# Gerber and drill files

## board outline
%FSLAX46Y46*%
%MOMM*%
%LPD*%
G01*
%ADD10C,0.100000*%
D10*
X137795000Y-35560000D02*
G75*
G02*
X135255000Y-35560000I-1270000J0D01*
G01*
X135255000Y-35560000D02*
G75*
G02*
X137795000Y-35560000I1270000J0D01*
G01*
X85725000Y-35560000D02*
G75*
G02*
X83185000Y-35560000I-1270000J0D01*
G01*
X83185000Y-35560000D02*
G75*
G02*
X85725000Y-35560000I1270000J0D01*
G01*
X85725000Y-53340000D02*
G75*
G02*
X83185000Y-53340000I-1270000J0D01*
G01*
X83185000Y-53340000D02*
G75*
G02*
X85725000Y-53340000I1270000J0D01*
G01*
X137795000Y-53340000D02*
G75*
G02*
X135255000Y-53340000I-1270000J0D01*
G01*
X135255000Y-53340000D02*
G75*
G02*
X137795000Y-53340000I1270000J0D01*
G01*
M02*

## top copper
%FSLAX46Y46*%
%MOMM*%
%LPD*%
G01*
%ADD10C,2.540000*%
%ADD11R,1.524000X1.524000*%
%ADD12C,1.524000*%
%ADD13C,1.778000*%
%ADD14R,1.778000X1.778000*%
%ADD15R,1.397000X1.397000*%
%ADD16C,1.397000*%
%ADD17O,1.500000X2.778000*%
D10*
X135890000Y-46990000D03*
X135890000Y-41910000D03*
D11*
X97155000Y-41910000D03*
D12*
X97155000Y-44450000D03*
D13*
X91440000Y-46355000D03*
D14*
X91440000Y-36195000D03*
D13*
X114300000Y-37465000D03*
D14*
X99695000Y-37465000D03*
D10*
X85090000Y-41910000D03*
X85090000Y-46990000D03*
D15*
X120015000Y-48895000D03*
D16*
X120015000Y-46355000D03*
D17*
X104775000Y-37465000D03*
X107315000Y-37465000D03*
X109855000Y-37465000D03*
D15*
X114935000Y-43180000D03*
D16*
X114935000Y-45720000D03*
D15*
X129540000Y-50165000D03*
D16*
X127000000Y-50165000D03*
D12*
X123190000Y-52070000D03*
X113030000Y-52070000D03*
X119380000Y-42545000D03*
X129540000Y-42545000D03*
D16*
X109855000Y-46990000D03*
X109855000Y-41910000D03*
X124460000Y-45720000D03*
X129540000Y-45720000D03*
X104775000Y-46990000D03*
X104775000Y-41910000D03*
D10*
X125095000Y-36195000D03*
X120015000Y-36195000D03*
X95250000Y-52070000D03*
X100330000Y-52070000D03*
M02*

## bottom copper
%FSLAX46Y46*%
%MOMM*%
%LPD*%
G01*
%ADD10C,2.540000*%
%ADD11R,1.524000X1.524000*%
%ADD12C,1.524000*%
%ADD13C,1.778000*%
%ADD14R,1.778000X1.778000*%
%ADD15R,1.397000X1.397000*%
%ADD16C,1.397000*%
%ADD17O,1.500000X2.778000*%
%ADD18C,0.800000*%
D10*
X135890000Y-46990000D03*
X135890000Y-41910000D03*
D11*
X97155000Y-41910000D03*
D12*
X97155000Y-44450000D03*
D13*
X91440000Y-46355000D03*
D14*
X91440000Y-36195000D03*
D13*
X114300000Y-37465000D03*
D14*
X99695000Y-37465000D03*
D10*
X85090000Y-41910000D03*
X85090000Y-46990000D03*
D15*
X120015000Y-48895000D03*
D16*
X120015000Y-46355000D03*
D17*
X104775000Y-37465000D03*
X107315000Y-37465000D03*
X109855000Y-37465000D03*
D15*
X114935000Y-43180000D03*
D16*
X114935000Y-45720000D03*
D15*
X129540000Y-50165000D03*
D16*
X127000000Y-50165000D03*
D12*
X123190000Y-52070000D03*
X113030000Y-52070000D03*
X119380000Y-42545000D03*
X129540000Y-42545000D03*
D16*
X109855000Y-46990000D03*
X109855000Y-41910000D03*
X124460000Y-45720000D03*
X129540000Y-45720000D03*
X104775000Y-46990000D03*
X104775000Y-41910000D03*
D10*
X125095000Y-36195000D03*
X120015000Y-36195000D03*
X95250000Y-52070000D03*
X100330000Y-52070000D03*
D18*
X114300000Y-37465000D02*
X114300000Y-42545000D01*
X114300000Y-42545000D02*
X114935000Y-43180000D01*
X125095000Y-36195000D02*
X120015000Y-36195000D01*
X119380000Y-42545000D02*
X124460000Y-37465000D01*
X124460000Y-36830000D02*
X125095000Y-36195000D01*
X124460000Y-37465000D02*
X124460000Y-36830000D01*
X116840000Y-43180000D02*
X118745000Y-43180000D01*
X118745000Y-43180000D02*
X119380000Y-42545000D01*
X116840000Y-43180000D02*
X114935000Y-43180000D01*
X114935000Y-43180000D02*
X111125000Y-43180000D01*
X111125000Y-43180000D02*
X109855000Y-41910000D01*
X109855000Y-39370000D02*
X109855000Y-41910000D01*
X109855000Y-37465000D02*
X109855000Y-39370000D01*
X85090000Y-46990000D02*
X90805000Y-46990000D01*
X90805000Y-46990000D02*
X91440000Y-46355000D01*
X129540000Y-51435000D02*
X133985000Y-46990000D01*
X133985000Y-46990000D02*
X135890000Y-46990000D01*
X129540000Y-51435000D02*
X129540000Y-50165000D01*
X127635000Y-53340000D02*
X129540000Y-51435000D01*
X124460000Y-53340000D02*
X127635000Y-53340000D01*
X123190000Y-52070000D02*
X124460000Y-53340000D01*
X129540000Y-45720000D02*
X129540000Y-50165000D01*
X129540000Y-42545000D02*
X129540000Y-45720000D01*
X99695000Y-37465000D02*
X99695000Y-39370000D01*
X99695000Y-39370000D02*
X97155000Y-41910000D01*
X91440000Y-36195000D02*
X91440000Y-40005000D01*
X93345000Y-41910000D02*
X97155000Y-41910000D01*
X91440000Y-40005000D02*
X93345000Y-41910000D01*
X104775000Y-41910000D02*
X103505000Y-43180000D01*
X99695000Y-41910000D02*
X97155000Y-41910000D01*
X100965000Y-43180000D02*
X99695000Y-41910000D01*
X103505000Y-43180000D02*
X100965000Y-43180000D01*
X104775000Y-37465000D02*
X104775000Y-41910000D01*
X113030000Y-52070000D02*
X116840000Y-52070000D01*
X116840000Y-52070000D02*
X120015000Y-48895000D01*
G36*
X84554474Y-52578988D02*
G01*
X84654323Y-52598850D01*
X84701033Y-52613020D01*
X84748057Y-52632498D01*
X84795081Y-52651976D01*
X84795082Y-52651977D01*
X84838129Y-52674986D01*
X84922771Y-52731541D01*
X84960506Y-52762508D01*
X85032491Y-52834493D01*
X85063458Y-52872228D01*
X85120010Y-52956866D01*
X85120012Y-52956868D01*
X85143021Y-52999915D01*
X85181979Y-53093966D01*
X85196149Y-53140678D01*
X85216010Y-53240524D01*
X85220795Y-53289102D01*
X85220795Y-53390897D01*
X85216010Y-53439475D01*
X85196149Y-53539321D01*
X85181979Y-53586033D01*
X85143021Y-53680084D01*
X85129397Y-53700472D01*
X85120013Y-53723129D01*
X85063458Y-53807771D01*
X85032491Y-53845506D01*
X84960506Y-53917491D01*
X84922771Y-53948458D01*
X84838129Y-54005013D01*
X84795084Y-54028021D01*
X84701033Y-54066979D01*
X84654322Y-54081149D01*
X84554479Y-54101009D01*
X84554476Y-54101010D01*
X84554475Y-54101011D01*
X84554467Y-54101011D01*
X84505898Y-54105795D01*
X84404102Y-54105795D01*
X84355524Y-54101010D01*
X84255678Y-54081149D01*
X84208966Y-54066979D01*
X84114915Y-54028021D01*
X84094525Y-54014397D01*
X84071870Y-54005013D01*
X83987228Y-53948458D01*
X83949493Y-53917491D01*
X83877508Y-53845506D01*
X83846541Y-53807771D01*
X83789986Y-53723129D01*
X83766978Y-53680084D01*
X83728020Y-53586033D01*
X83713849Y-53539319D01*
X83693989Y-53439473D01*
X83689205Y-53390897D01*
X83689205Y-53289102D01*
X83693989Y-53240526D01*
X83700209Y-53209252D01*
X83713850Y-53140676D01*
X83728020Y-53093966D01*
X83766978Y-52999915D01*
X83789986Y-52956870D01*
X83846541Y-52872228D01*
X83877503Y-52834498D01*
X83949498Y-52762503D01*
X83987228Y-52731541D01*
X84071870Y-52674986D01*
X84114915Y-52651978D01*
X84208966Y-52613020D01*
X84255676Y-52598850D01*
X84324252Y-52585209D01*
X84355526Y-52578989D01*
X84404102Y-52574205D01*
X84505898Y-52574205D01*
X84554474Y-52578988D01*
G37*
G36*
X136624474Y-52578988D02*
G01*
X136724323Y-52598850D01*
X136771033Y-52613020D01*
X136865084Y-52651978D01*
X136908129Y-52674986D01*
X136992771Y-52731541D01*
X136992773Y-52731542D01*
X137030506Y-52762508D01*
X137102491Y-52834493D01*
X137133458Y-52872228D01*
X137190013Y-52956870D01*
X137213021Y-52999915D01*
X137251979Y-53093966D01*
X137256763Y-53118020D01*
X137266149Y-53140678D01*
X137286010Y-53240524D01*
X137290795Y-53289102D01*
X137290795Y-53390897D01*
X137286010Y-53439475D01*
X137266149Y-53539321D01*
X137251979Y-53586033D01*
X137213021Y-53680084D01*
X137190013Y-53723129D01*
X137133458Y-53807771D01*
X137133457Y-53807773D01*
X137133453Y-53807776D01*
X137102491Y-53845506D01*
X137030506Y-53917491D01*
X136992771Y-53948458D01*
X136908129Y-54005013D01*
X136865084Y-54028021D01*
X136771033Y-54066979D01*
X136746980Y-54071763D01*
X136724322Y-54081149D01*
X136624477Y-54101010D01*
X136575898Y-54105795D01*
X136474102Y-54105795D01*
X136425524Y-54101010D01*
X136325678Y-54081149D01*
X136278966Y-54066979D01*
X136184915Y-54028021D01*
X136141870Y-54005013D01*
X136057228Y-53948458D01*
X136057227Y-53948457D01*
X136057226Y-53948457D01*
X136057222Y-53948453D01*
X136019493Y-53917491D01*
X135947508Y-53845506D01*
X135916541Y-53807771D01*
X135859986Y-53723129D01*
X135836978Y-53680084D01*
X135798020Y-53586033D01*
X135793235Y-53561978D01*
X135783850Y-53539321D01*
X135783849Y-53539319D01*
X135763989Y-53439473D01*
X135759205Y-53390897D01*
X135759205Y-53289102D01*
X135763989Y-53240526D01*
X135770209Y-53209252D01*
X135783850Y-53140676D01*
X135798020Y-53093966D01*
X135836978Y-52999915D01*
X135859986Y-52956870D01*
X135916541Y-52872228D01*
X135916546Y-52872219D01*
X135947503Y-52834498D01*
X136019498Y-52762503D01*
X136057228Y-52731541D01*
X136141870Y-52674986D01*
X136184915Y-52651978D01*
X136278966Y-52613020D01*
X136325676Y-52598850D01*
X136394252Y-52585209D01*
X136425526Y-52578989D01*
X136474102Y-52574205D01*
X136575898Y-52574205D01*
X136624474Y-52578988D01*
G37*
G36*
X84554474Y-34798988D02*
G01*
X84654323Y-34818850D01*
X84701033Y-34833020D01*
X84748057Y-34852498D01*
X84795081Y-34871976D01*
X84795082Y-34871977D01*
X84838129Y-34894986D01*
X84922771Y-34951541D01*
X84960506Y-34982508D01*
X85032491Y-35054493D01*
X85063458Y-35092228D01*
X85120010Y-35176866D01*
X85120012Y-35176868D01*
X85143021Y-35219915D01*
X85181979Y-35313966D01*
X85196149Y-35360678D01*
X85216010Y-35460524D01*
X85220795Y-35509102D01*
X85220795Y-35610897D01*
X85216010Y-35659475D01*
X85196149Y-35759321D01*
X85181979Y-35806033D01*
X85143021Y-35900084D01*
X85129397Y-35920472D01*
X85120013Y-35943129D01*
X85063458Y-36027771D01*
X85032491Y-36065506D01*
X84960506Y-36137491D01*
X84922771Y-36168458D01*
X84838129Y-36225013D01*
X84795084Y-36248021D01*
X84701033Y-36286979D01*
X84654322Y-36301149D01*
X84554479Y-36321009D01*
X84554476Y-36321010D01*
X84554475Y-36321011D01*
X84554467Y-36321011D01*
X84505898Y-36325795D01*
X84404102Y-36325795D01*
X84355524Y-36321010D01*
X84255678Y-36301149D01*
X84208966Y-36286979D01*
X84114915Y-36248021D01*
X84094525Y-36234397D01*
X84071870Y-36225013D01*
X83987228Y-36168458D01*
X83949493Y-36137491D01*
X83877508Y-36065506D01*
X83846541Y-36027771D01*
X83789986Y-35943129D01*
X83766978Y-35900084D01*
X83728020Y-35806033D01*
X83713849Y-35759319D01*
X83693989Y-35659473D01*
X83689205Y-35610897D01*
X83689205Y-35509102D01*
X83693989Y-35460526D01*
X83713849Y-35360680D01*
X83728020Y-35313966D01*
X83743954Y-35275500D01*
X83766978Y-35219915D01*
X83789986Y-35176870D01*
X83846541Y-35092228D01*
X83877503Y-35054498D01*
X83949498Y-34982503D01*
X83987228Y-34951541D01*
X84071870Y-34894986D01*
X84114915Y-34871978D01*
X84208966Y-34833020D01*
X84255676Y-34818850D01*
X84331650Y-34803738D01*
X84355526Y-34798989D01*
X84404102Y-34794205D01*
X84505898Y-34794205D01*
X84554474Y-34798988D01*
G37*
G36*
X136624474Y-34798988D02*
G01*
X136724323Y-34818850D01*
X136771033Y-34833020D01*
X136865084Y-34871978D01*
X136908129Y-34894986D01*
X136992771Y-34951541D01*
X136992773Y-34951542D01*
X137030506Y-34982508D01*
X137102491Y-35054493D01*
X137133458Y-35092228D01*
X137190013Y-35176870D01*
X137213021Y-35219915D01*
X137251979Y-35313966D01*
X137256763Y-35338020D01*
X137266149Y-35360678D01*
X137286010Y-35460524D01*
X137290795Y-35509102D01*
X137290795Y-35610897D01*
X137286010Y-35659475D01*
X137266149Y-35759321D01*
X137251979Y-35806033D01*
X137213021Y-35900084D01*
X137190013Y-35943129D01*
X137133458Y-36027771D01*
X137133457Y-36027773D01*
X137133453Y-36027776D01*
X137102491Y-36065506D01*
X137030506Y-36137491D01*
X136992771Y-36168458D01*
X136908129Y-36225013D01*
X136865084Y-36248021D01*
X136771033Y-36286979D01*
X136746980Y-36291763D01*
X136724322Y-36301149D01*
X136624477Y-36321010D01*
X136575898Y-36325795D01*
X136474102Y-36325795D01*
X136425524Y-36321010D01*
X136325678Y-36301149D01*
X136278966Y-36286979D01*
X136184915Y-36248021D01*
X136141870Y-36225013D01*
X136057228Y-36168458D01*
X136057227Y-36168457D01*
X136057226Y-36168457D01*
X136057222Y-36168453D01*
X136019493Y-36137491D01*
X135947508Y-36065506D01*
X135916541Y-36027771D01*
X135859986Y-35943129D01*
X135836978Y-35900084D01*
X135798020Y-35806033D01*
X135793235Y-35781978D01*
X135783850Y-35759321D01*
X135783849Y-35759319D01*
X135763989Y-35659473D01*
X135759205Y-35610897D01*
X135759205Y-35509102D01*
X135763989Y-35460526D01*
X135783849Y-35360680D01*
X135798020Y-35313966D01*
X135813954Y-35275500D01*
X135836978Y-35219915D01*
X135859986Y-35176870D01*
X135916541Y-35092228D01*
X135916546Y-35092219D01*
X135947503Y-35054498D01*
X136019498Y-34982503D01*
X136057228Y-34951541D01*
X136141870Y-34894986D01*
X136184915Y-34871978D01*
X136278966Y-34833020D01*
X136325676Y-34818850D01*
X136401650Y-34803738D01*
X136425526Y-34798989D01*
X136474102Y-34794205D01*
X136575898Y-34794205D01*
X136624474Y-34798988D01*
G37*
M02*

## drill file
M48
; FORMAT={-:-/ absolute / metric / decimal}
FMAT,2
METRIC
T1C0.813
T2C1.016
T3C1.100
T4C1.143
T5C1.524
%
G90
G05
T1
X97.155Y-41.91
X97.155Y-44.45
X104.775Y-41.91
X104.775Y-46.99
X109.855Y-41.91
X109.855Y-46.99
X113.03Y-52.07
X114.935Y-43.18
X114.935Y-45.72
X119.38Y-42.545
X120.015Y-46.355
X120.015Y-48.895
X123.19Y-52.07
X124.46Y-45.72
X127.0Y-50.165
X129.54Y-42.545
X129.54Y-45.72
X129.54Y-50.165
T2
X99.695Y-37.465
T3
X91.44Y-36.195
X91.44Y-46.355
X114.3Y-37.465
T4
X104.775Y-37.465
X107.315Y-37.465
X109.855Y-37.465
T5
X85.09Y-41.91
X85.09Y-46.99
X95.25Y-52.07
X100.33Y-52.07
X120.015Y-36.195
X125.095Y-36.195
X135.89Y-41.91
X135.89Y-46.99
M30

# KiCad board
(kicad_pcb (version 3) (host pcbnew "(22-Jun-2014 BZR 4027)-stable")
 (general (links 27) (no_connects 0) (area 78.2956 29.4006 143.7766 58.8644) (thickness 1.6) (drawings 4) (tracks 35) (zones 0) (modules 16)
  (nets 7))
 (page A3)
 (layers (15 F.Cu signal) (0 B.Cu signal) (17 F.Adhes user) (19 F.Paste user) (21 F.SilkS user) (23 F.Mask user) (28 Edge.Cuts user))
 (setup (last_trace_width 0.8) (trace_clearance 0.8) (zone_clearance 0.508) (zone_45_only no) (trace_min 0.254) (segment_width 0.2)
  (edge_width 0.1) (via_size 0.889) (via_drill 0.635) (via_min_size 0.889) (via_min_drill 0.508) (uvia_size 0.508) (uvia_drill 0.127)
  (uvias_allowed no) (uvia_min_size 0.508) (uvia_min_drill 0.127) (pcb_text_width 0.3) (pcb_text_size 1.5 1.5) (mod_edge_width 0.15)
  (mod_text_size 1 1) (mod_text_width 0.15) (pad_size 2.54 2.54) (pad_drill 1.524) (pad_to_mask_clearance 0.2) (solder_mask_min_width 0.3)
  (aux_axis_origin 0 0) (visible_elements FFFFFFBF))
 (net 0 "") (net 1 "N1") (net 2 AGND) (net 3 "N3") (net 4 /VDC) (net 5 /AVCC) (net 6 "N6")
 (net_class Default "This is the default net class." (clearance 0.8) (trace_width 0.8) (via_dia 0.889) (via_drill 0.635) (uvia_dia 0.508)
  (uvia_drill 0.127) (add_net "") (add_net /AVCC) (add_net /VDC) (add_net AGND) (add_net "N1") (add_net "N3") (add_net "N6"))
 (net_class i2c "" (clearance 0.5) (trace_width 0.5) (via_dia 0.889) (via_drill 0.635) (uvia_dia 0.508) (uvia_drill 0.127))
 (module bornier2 (layer F.Cu) (at 135.89 44.45 90)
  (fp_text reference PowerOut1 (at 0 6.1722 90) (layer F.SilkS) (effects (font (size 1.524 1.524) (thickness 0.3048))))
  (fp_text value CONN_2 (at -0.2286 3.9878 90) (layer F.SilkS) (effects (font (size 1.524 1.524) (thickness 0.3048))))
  (pad 1 thru_hole circle (at -2.54 0 90) (size 2.54 2.54) (drill 1.524) (layers *.Cu *.Mask F.SilkS) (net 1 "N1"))
  (pad 2 thru_hole circle (at 2.54 0 90) (size 2.54 2.54) (drill 1.524) (layers *.Cu *.Mask F.SilkS) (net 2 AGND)))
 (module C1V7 (layer F.Cu) (at 97.155 43.18 270)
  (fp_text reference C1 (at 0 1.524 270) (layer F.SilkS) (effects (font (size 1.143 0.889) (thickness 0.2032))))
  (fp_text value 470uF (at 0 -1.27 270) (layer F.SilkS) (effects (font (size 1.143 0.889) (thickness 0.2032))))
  (pad 1 thru_hole rect (at -1.27 0 270) (size 1.524 1.524) (drill 0.8128) (layers *.Cu *.Mask F.SilkS) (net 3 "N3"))
  (pad 2 thru_hole circle (at 1.27 0 270) (size 1.524 1.524) (drill 0.8128) (layers *.Cu *.Mask F.SilkS) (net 2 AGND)))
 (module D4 (layer F.Cu) (at 91.44 41.275 90)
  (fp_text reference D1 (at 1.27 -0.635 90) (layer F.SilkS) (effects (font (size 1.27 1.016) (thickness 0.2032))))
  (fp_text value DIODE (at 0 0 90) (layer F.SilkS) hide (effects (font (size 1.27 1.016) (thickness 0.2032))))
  (pad 1 thru_hole circle (at -5.08 0 90) (size 1.778 1.778) (drill 1.1) (layers *.Cu *.Mask F.SilkS) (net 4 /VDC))
  (pad 2 thru_hole rect (at 5.08 0 90) (size 1.778 1.778) (drill 1.1) (layers *.Cu *.Mask F.SilkS) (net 3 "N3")))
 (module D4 (layer F.Cu) (at 107.315 37.465 180)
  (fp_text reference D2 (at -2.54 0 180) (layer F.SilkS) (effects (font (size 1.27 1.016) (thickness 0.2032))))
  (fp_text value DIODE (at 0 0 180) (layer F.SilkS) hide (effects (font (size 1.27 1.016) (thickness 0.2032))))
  (pad 1 thru_hole circle (at -6.985 0 180) (size 1.778 1.778) (drill 1.1) (layers *.Cu *.Mask F.SilkS) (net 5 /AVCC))
  (pad 2 thru_hole rect (at 7.62 0 180) (size 1.778 1.778) (drill 1.016) (layers *.Cu *.Mask F.SilkS) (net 3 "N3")))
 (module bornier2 (layer F.Cu) (at 85.09 44.45 270)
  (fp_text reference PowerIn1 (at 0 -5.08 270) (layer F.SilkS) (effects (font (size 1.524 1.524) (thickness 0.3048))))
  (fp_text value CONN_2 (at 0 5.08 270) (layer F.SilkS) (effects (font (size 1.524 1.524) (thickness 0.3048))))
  (pad 1 thru_hole circle (at -2.54 0 270) (size 2.54 2.54) (drill 1.524) (layers *.Cu *.Mask F.SilkS) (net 2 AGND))
  (pad 2 thru_hole circle (at 2.54 0 270) (size 2.54 2.54) (drill 1.524) (layers *.Cu *.Mask F.SilkS) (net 4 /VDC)))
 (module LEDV (layer F.Cu) (at 120.015 47.625 90)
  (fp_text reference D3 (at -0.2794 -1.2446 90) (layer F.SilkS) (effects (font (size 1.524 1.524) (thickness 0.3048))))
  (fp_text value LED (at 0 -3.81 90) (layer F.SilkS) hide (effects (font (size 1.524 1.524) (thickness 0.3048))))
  (pad 1 thru_hole rect (at -1.27 0 90) (size 1.397 1.397) (drill 0.8128) (layers *.Cu *.Mask F.SilkS) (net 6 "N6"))
  (pad 2 thru_hole circle (at 1.27 0 90) (size 1.397 1.397) (drill 0.8128) (layers *.Cu *.Mask F.SilkS) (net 2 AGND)))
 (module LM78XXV (layer B.Cu) (at 107.315 37.465 270)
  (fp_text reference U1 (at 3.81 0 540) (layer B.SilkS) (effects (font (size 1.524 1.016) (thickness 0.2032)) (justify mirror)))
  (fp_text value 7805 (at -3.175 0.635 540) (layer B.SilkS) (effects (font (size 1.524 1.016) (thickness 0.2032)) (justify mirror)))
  (pad VI thru_hole oval (at 0 2.54 270) (size 2.778 1.5) (drill 1.143) (layers *.Cu *.Mask) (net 3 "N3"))
  (pad GND thru_hole oval (at 0 0 270) (size 2.778 1.5) (drill 1.143) (layers *.Cu *.Mask) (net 2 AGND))
  (pad VO thru_hole oval (at 0 -2.54 270) (size 2.778 1.5) (drill 1.143) (layers *.Cu *.Mask) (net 5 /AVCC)))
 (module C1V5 (layer F.Cu) (at 114.935 44.45 270)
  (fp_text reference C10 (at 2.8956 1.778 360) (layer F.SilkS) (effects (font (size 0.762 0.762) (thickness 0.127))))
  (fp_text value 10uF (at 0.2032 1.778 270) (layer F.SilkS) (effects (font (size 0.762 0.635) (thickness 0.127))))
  (pad 1 thru_hole rect (at -1.27 0 270) (size 1.397 1.397) (drill 0.8128) (layers *.Cu *.Mask F.SilkS) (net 5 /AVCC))
  (pad 2 thru_hole circle (at 1.27 0 270) (size 1.397 1.397) (drill 0.8128) (layers *.Cu *.Mask F.SilkS) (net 2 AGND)))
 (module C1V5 (layer F.Cu) (at 128.27 50.165 180)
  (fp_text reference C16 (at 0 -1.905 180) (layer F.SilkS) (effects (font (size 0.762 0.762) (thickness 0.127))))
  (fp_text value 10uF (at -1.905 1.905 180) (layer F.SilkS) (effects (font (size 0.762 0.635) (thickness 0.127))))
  (pad 1 thru_hole rect (at -1.27 0 180) (size 1.397 1.397) (drill 0.8128) (layers *.Cu *.Mask F.SilkS) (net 1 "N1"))
  (pad 2 thru_hole circle (at 1.27 0 180) (size 1.397 1.397) (drill 0.8128) (layers *.Cu *.Mask F.SilkS) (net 2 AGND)))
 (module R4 (layer F.Cu) (at 118.11 52.07 180) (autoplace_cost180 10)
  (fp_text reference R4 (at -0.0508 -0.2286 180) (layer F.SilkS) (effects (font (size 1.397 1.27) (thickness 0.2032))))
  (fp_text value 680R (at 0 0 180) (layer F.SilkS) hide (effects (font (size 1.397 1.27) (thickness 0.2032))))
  (pad 1 thru_hole circle (at -5.08 0 180) (size 1.524 1.524) (drill 0.8128) (layers *.Cu *.Mask F.SilkS) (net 1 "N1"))
  (pad 2 thru_hole circle (at 5.08 0 180) (size 1.524 1.524) (drill 0.8128) (layers *.Cu *.Mask F.SilkS) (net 6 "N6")))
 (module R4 (layer F.Cu) (at 124.46 42.545) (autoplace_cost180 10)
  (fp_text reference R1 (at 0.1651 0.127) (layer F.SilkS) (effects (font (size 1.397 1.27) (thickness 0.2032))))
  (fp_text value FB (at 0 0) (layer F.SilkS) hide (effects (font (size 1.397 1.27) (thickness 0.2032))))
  (pad 1 thru_hole circle (at -5.08 0) (size 1.524 1.524) (drill 0.8128) (layers *.Cu *.Mask F.SilkS) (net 5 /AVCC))
  (pad 2 thru_hole circle (at 5.08 0) (size 1.524 1.524) (drill 0.8128) (layers *.Cu *.Mask F.SilkS) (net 1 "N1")))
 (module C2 (layer F.Cu) (at 109.855 44.45 90)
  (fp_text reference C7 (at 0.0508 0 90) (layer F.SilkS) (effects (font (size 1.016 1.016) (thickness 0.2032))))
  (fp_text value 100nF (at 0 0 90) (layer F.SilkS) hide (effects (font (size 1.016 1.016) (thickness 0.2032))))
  (pad 1 thru_hole circle (at -2.54 0 90) (size 1.397 1.397) (drill 0.8128) (layers *.Cu *.Mask F.SilkS) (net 2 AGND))
  (pad 2 thru_hole circle (at 2.54 0 90) (size 1.397 1.397) (drill 0.8128) (layers *.Cu *.Mask F.SilkS) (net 5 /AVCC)))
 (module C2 (layer F.Cu) (at 127 45.72)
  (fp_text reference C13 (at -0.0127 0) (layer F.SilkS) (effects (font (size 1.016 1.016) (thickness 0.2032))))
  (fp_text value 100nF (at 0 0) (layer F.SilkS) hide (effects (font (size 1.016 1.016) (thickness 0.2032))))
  (pad 1 thru_hole circle (at -2.54 0) (size 1.397 1.397) (drill 0.8128) (layers *.Cu *.Mask F.SilkS) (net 2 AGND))
  (pad 2 thru_hole circle (at 2.54 0) (size 1.397 1.397) (drill 0.8128) (layers *.Cu *.Mask F.SilkS) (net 1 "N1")))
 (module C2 (layer F.Cu) (at 104.775 44.45 90)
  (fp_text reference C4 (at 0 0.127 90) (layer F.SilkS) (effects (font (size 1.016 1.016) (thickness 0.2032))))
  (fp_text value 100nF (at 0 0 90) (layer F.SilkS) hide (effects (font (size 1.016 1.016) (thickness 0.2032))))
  (pad 1 thru_hole circle (at -2.54 0 90) (size 1.397 1.397) (drill 0.8128) (layers *.Cu *.Mask F.SilkS) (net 2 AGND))
  (pad 2 thru_hole circle (at 2.54 0 90) (size 1.397 1.397) (drill 0.8128) (layers *.Cu *.Mask F.SilkS) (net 3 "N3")))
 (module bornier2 (layer F.Cu) (at 122.555 36.195 180)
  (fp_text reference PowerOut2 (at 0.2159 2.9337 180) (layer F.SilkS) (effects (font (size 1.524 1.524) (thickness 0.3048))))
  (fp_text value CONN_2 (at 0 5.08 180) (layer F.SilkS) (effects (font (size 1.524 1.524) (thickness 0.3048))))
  (pad 1 thru_hole circle (at -2.54 0 180) (size 2.54 2.54) (drill 1.524) (layers *.Cu *.Mask F.SilkS) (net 5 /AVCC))
  (pad 2 thru_hole circle (at 2.54 0 180) (size 2.54 2.54) (drill 1.524) (layers *.Cu *.Mask F.SilkS) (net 5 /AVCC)))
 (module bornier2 (layer F.Cu) (at 97.79 52.07)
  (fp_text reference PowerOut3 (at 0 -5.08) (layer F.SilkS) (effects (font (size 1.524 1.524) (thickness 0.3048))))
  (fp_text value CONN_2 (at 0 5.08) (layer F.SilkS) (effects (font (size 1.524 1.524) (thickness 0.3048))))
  (pad 1 thru_hole circle (at -2.54 0) (size 2.54 2.54) (drill 1.524) (layers *.Cu *.Mask F.SilkS) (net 2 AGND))
  (pad 2 thru_hole circle (at 2.54 0) (size 2.54 2.54) (drill 1.524) (layers *.Cu *.Mask F.SilkS) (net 2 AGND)))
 (gr_circle (center 136.525 35.56) (end 137.795 35.56) (layer Edge.Cuts) (width 0.1))
 (gr_circle (center 84.455 35.56) (end 85.725 35.56) (layer Edge.Cuts) (width 0.1))
 (gr_circle (center 84.455 53.34) (end 85.725 53.34) (layer Edge.Cuts) (width 0.1))
 (gr_circle (center 136.525 53.34) (end 137.795 53.34) (layer Edge.Cuts) (width 0.1))
 (segment (start 114.3 37.465) (end 114.3 42.545) (width 0.8) (layer B.Cu) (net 5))
 (segment (start 114.3 42.545) (end 114.935 43.18) (width 0.8) (layer B.Cu) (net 5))
 (segment (start 125.095 36.195) (end 120.015 36.195) (width 0.8) (layer B.Cu) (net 5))
 (segment (start 119.38 42.545) (end 124.46 37.465) (width 0.8) (layer B.Cu) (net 5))
 (segment (start 124.46 36.83) (end 125.095 36.195) (width 0.8) (layer B.Cu) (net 5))
 (segment (start 124.46 37.465) (end 124.46 36.83) (width 0.8) (layer B.Cu) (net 5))
 (segment (start 116.84 43.18) (end 118.745 43.18) (width 0.8) (layer B.Cu) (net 5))
 (segment (start 118.745 43.18) (end 119.38 42.545) (width 0.8) (layer B.Cu) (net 5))
 (segment (start 116.84 43.18) (end 114.935 43.18) (width 0.8) (layer B.Cu) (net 5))
 (segment (start 114.935 43.18) (end 111.125 43.18) (width 0.8) (layer B.Cu) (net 5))
 (segment (start 111.125 43.18) (end 109.855 41.91) (width 0.8) (layer B.Cu) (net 5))
 (segment (start 109.855 39.37) (end 109.855 41.91) (width 0.8) (layer B.Cu) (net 5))
 (segment (start 109.855 37.465) (end 109.855 39.37) (width 0.8) (layer B.Cu) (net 5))
 (segment (start 85.09 46.99) (end 90.805 46.99) (width 0.8) (layer B.Cu) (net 4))
 (segment (start 90.805 46.99) (end 91.44 46.355) (width 0.8) (layer B.Cu) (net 4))
 (segment (start 129.54 51.435) (end 133.985 46.99) (width 0.8) (layer B.Cu) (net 1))
 (segment (start 133.985 46.99) (end 135.89 46.99) (width 0.8) (layer B.Cu) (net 1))
 (segment (start 129.54 51.435) (end 129.54 50.165) (width 0.8) (layer B.Cu) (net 1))
 (segment (start 127.635 53.34) (end 129.54 51.435) (width 0.8) (layer B.Cu) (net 1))
 (segment (start 124.46 53.34) (end 127.635 53.34) (width 0.8) (layer B.Cu) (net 1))
 (segment (start 123.19 52.07) (end 124.46 53.34) (width 0.8) (layer B.Cu) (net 1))
 (segment (start 129.54 45.72) (end 129.54 50.165) (width 0.8) (layer B.Cu) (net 1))
 (segment (start 129.54 42.545) (end 129.54 45.72) (width 0.8) (layer B.Cu) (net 1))
 (segment (start 99.695 37.465) (end 99.695 39.37) (width 0.8) (layer B.Cu) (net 3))
 (segment (start 99.695 39.37) (end 97.155 41.91) (width 0.8) (layer B.Cu) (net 3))
 (segment (start 91.44 36.195) (end 91.44 40.005) (width 0.8) (layer B.Cu) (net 3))
 (segment (start 93.345 41.91) (end 97.155 41.91) (width 0.8) (layer B.Cu) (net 3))
 (segment (start 91.44 40.005) (end 93.345 41.91) (width 0.8) (layer B.Cu) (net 3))
 (segment (start 104.775 41.91) (end 103.505 43.18) (width 0.8) (layer B.Cu) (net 3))
 (segment (start 99.695 41.91) (end 97.155 41.91) (width 0.8) (layer B.Cu) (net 3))
 (segment (start 100.965 43.18) (end 99.695 41.91) (width 0.8) (layer B.Cu) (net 3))
 (segment (start 103.505 43.18) (end 100.965 43.18) (width 0.8) (layer B.Cu) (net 3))
 (segment (start 104.775 37.465) (end 104.775 41.91) (width 0.8) (layer B.Cu) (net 3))
 (segment (start 113.03 52.07) (end 116.84 52.07) (width 0.8) (layer B.Cu) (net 6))
 (segment (start 116.84 52.07) (end 120.015 48.895) (width 0.8) (layer B.Cu) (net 6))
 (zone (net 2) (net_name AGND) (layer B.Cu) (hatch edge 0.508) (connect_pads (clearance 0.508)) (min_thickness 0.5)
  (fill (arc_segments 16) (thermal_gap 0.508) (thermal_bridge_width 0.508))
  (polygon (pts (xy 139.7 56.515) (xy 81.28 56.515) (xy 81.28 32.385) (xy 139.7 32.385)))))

